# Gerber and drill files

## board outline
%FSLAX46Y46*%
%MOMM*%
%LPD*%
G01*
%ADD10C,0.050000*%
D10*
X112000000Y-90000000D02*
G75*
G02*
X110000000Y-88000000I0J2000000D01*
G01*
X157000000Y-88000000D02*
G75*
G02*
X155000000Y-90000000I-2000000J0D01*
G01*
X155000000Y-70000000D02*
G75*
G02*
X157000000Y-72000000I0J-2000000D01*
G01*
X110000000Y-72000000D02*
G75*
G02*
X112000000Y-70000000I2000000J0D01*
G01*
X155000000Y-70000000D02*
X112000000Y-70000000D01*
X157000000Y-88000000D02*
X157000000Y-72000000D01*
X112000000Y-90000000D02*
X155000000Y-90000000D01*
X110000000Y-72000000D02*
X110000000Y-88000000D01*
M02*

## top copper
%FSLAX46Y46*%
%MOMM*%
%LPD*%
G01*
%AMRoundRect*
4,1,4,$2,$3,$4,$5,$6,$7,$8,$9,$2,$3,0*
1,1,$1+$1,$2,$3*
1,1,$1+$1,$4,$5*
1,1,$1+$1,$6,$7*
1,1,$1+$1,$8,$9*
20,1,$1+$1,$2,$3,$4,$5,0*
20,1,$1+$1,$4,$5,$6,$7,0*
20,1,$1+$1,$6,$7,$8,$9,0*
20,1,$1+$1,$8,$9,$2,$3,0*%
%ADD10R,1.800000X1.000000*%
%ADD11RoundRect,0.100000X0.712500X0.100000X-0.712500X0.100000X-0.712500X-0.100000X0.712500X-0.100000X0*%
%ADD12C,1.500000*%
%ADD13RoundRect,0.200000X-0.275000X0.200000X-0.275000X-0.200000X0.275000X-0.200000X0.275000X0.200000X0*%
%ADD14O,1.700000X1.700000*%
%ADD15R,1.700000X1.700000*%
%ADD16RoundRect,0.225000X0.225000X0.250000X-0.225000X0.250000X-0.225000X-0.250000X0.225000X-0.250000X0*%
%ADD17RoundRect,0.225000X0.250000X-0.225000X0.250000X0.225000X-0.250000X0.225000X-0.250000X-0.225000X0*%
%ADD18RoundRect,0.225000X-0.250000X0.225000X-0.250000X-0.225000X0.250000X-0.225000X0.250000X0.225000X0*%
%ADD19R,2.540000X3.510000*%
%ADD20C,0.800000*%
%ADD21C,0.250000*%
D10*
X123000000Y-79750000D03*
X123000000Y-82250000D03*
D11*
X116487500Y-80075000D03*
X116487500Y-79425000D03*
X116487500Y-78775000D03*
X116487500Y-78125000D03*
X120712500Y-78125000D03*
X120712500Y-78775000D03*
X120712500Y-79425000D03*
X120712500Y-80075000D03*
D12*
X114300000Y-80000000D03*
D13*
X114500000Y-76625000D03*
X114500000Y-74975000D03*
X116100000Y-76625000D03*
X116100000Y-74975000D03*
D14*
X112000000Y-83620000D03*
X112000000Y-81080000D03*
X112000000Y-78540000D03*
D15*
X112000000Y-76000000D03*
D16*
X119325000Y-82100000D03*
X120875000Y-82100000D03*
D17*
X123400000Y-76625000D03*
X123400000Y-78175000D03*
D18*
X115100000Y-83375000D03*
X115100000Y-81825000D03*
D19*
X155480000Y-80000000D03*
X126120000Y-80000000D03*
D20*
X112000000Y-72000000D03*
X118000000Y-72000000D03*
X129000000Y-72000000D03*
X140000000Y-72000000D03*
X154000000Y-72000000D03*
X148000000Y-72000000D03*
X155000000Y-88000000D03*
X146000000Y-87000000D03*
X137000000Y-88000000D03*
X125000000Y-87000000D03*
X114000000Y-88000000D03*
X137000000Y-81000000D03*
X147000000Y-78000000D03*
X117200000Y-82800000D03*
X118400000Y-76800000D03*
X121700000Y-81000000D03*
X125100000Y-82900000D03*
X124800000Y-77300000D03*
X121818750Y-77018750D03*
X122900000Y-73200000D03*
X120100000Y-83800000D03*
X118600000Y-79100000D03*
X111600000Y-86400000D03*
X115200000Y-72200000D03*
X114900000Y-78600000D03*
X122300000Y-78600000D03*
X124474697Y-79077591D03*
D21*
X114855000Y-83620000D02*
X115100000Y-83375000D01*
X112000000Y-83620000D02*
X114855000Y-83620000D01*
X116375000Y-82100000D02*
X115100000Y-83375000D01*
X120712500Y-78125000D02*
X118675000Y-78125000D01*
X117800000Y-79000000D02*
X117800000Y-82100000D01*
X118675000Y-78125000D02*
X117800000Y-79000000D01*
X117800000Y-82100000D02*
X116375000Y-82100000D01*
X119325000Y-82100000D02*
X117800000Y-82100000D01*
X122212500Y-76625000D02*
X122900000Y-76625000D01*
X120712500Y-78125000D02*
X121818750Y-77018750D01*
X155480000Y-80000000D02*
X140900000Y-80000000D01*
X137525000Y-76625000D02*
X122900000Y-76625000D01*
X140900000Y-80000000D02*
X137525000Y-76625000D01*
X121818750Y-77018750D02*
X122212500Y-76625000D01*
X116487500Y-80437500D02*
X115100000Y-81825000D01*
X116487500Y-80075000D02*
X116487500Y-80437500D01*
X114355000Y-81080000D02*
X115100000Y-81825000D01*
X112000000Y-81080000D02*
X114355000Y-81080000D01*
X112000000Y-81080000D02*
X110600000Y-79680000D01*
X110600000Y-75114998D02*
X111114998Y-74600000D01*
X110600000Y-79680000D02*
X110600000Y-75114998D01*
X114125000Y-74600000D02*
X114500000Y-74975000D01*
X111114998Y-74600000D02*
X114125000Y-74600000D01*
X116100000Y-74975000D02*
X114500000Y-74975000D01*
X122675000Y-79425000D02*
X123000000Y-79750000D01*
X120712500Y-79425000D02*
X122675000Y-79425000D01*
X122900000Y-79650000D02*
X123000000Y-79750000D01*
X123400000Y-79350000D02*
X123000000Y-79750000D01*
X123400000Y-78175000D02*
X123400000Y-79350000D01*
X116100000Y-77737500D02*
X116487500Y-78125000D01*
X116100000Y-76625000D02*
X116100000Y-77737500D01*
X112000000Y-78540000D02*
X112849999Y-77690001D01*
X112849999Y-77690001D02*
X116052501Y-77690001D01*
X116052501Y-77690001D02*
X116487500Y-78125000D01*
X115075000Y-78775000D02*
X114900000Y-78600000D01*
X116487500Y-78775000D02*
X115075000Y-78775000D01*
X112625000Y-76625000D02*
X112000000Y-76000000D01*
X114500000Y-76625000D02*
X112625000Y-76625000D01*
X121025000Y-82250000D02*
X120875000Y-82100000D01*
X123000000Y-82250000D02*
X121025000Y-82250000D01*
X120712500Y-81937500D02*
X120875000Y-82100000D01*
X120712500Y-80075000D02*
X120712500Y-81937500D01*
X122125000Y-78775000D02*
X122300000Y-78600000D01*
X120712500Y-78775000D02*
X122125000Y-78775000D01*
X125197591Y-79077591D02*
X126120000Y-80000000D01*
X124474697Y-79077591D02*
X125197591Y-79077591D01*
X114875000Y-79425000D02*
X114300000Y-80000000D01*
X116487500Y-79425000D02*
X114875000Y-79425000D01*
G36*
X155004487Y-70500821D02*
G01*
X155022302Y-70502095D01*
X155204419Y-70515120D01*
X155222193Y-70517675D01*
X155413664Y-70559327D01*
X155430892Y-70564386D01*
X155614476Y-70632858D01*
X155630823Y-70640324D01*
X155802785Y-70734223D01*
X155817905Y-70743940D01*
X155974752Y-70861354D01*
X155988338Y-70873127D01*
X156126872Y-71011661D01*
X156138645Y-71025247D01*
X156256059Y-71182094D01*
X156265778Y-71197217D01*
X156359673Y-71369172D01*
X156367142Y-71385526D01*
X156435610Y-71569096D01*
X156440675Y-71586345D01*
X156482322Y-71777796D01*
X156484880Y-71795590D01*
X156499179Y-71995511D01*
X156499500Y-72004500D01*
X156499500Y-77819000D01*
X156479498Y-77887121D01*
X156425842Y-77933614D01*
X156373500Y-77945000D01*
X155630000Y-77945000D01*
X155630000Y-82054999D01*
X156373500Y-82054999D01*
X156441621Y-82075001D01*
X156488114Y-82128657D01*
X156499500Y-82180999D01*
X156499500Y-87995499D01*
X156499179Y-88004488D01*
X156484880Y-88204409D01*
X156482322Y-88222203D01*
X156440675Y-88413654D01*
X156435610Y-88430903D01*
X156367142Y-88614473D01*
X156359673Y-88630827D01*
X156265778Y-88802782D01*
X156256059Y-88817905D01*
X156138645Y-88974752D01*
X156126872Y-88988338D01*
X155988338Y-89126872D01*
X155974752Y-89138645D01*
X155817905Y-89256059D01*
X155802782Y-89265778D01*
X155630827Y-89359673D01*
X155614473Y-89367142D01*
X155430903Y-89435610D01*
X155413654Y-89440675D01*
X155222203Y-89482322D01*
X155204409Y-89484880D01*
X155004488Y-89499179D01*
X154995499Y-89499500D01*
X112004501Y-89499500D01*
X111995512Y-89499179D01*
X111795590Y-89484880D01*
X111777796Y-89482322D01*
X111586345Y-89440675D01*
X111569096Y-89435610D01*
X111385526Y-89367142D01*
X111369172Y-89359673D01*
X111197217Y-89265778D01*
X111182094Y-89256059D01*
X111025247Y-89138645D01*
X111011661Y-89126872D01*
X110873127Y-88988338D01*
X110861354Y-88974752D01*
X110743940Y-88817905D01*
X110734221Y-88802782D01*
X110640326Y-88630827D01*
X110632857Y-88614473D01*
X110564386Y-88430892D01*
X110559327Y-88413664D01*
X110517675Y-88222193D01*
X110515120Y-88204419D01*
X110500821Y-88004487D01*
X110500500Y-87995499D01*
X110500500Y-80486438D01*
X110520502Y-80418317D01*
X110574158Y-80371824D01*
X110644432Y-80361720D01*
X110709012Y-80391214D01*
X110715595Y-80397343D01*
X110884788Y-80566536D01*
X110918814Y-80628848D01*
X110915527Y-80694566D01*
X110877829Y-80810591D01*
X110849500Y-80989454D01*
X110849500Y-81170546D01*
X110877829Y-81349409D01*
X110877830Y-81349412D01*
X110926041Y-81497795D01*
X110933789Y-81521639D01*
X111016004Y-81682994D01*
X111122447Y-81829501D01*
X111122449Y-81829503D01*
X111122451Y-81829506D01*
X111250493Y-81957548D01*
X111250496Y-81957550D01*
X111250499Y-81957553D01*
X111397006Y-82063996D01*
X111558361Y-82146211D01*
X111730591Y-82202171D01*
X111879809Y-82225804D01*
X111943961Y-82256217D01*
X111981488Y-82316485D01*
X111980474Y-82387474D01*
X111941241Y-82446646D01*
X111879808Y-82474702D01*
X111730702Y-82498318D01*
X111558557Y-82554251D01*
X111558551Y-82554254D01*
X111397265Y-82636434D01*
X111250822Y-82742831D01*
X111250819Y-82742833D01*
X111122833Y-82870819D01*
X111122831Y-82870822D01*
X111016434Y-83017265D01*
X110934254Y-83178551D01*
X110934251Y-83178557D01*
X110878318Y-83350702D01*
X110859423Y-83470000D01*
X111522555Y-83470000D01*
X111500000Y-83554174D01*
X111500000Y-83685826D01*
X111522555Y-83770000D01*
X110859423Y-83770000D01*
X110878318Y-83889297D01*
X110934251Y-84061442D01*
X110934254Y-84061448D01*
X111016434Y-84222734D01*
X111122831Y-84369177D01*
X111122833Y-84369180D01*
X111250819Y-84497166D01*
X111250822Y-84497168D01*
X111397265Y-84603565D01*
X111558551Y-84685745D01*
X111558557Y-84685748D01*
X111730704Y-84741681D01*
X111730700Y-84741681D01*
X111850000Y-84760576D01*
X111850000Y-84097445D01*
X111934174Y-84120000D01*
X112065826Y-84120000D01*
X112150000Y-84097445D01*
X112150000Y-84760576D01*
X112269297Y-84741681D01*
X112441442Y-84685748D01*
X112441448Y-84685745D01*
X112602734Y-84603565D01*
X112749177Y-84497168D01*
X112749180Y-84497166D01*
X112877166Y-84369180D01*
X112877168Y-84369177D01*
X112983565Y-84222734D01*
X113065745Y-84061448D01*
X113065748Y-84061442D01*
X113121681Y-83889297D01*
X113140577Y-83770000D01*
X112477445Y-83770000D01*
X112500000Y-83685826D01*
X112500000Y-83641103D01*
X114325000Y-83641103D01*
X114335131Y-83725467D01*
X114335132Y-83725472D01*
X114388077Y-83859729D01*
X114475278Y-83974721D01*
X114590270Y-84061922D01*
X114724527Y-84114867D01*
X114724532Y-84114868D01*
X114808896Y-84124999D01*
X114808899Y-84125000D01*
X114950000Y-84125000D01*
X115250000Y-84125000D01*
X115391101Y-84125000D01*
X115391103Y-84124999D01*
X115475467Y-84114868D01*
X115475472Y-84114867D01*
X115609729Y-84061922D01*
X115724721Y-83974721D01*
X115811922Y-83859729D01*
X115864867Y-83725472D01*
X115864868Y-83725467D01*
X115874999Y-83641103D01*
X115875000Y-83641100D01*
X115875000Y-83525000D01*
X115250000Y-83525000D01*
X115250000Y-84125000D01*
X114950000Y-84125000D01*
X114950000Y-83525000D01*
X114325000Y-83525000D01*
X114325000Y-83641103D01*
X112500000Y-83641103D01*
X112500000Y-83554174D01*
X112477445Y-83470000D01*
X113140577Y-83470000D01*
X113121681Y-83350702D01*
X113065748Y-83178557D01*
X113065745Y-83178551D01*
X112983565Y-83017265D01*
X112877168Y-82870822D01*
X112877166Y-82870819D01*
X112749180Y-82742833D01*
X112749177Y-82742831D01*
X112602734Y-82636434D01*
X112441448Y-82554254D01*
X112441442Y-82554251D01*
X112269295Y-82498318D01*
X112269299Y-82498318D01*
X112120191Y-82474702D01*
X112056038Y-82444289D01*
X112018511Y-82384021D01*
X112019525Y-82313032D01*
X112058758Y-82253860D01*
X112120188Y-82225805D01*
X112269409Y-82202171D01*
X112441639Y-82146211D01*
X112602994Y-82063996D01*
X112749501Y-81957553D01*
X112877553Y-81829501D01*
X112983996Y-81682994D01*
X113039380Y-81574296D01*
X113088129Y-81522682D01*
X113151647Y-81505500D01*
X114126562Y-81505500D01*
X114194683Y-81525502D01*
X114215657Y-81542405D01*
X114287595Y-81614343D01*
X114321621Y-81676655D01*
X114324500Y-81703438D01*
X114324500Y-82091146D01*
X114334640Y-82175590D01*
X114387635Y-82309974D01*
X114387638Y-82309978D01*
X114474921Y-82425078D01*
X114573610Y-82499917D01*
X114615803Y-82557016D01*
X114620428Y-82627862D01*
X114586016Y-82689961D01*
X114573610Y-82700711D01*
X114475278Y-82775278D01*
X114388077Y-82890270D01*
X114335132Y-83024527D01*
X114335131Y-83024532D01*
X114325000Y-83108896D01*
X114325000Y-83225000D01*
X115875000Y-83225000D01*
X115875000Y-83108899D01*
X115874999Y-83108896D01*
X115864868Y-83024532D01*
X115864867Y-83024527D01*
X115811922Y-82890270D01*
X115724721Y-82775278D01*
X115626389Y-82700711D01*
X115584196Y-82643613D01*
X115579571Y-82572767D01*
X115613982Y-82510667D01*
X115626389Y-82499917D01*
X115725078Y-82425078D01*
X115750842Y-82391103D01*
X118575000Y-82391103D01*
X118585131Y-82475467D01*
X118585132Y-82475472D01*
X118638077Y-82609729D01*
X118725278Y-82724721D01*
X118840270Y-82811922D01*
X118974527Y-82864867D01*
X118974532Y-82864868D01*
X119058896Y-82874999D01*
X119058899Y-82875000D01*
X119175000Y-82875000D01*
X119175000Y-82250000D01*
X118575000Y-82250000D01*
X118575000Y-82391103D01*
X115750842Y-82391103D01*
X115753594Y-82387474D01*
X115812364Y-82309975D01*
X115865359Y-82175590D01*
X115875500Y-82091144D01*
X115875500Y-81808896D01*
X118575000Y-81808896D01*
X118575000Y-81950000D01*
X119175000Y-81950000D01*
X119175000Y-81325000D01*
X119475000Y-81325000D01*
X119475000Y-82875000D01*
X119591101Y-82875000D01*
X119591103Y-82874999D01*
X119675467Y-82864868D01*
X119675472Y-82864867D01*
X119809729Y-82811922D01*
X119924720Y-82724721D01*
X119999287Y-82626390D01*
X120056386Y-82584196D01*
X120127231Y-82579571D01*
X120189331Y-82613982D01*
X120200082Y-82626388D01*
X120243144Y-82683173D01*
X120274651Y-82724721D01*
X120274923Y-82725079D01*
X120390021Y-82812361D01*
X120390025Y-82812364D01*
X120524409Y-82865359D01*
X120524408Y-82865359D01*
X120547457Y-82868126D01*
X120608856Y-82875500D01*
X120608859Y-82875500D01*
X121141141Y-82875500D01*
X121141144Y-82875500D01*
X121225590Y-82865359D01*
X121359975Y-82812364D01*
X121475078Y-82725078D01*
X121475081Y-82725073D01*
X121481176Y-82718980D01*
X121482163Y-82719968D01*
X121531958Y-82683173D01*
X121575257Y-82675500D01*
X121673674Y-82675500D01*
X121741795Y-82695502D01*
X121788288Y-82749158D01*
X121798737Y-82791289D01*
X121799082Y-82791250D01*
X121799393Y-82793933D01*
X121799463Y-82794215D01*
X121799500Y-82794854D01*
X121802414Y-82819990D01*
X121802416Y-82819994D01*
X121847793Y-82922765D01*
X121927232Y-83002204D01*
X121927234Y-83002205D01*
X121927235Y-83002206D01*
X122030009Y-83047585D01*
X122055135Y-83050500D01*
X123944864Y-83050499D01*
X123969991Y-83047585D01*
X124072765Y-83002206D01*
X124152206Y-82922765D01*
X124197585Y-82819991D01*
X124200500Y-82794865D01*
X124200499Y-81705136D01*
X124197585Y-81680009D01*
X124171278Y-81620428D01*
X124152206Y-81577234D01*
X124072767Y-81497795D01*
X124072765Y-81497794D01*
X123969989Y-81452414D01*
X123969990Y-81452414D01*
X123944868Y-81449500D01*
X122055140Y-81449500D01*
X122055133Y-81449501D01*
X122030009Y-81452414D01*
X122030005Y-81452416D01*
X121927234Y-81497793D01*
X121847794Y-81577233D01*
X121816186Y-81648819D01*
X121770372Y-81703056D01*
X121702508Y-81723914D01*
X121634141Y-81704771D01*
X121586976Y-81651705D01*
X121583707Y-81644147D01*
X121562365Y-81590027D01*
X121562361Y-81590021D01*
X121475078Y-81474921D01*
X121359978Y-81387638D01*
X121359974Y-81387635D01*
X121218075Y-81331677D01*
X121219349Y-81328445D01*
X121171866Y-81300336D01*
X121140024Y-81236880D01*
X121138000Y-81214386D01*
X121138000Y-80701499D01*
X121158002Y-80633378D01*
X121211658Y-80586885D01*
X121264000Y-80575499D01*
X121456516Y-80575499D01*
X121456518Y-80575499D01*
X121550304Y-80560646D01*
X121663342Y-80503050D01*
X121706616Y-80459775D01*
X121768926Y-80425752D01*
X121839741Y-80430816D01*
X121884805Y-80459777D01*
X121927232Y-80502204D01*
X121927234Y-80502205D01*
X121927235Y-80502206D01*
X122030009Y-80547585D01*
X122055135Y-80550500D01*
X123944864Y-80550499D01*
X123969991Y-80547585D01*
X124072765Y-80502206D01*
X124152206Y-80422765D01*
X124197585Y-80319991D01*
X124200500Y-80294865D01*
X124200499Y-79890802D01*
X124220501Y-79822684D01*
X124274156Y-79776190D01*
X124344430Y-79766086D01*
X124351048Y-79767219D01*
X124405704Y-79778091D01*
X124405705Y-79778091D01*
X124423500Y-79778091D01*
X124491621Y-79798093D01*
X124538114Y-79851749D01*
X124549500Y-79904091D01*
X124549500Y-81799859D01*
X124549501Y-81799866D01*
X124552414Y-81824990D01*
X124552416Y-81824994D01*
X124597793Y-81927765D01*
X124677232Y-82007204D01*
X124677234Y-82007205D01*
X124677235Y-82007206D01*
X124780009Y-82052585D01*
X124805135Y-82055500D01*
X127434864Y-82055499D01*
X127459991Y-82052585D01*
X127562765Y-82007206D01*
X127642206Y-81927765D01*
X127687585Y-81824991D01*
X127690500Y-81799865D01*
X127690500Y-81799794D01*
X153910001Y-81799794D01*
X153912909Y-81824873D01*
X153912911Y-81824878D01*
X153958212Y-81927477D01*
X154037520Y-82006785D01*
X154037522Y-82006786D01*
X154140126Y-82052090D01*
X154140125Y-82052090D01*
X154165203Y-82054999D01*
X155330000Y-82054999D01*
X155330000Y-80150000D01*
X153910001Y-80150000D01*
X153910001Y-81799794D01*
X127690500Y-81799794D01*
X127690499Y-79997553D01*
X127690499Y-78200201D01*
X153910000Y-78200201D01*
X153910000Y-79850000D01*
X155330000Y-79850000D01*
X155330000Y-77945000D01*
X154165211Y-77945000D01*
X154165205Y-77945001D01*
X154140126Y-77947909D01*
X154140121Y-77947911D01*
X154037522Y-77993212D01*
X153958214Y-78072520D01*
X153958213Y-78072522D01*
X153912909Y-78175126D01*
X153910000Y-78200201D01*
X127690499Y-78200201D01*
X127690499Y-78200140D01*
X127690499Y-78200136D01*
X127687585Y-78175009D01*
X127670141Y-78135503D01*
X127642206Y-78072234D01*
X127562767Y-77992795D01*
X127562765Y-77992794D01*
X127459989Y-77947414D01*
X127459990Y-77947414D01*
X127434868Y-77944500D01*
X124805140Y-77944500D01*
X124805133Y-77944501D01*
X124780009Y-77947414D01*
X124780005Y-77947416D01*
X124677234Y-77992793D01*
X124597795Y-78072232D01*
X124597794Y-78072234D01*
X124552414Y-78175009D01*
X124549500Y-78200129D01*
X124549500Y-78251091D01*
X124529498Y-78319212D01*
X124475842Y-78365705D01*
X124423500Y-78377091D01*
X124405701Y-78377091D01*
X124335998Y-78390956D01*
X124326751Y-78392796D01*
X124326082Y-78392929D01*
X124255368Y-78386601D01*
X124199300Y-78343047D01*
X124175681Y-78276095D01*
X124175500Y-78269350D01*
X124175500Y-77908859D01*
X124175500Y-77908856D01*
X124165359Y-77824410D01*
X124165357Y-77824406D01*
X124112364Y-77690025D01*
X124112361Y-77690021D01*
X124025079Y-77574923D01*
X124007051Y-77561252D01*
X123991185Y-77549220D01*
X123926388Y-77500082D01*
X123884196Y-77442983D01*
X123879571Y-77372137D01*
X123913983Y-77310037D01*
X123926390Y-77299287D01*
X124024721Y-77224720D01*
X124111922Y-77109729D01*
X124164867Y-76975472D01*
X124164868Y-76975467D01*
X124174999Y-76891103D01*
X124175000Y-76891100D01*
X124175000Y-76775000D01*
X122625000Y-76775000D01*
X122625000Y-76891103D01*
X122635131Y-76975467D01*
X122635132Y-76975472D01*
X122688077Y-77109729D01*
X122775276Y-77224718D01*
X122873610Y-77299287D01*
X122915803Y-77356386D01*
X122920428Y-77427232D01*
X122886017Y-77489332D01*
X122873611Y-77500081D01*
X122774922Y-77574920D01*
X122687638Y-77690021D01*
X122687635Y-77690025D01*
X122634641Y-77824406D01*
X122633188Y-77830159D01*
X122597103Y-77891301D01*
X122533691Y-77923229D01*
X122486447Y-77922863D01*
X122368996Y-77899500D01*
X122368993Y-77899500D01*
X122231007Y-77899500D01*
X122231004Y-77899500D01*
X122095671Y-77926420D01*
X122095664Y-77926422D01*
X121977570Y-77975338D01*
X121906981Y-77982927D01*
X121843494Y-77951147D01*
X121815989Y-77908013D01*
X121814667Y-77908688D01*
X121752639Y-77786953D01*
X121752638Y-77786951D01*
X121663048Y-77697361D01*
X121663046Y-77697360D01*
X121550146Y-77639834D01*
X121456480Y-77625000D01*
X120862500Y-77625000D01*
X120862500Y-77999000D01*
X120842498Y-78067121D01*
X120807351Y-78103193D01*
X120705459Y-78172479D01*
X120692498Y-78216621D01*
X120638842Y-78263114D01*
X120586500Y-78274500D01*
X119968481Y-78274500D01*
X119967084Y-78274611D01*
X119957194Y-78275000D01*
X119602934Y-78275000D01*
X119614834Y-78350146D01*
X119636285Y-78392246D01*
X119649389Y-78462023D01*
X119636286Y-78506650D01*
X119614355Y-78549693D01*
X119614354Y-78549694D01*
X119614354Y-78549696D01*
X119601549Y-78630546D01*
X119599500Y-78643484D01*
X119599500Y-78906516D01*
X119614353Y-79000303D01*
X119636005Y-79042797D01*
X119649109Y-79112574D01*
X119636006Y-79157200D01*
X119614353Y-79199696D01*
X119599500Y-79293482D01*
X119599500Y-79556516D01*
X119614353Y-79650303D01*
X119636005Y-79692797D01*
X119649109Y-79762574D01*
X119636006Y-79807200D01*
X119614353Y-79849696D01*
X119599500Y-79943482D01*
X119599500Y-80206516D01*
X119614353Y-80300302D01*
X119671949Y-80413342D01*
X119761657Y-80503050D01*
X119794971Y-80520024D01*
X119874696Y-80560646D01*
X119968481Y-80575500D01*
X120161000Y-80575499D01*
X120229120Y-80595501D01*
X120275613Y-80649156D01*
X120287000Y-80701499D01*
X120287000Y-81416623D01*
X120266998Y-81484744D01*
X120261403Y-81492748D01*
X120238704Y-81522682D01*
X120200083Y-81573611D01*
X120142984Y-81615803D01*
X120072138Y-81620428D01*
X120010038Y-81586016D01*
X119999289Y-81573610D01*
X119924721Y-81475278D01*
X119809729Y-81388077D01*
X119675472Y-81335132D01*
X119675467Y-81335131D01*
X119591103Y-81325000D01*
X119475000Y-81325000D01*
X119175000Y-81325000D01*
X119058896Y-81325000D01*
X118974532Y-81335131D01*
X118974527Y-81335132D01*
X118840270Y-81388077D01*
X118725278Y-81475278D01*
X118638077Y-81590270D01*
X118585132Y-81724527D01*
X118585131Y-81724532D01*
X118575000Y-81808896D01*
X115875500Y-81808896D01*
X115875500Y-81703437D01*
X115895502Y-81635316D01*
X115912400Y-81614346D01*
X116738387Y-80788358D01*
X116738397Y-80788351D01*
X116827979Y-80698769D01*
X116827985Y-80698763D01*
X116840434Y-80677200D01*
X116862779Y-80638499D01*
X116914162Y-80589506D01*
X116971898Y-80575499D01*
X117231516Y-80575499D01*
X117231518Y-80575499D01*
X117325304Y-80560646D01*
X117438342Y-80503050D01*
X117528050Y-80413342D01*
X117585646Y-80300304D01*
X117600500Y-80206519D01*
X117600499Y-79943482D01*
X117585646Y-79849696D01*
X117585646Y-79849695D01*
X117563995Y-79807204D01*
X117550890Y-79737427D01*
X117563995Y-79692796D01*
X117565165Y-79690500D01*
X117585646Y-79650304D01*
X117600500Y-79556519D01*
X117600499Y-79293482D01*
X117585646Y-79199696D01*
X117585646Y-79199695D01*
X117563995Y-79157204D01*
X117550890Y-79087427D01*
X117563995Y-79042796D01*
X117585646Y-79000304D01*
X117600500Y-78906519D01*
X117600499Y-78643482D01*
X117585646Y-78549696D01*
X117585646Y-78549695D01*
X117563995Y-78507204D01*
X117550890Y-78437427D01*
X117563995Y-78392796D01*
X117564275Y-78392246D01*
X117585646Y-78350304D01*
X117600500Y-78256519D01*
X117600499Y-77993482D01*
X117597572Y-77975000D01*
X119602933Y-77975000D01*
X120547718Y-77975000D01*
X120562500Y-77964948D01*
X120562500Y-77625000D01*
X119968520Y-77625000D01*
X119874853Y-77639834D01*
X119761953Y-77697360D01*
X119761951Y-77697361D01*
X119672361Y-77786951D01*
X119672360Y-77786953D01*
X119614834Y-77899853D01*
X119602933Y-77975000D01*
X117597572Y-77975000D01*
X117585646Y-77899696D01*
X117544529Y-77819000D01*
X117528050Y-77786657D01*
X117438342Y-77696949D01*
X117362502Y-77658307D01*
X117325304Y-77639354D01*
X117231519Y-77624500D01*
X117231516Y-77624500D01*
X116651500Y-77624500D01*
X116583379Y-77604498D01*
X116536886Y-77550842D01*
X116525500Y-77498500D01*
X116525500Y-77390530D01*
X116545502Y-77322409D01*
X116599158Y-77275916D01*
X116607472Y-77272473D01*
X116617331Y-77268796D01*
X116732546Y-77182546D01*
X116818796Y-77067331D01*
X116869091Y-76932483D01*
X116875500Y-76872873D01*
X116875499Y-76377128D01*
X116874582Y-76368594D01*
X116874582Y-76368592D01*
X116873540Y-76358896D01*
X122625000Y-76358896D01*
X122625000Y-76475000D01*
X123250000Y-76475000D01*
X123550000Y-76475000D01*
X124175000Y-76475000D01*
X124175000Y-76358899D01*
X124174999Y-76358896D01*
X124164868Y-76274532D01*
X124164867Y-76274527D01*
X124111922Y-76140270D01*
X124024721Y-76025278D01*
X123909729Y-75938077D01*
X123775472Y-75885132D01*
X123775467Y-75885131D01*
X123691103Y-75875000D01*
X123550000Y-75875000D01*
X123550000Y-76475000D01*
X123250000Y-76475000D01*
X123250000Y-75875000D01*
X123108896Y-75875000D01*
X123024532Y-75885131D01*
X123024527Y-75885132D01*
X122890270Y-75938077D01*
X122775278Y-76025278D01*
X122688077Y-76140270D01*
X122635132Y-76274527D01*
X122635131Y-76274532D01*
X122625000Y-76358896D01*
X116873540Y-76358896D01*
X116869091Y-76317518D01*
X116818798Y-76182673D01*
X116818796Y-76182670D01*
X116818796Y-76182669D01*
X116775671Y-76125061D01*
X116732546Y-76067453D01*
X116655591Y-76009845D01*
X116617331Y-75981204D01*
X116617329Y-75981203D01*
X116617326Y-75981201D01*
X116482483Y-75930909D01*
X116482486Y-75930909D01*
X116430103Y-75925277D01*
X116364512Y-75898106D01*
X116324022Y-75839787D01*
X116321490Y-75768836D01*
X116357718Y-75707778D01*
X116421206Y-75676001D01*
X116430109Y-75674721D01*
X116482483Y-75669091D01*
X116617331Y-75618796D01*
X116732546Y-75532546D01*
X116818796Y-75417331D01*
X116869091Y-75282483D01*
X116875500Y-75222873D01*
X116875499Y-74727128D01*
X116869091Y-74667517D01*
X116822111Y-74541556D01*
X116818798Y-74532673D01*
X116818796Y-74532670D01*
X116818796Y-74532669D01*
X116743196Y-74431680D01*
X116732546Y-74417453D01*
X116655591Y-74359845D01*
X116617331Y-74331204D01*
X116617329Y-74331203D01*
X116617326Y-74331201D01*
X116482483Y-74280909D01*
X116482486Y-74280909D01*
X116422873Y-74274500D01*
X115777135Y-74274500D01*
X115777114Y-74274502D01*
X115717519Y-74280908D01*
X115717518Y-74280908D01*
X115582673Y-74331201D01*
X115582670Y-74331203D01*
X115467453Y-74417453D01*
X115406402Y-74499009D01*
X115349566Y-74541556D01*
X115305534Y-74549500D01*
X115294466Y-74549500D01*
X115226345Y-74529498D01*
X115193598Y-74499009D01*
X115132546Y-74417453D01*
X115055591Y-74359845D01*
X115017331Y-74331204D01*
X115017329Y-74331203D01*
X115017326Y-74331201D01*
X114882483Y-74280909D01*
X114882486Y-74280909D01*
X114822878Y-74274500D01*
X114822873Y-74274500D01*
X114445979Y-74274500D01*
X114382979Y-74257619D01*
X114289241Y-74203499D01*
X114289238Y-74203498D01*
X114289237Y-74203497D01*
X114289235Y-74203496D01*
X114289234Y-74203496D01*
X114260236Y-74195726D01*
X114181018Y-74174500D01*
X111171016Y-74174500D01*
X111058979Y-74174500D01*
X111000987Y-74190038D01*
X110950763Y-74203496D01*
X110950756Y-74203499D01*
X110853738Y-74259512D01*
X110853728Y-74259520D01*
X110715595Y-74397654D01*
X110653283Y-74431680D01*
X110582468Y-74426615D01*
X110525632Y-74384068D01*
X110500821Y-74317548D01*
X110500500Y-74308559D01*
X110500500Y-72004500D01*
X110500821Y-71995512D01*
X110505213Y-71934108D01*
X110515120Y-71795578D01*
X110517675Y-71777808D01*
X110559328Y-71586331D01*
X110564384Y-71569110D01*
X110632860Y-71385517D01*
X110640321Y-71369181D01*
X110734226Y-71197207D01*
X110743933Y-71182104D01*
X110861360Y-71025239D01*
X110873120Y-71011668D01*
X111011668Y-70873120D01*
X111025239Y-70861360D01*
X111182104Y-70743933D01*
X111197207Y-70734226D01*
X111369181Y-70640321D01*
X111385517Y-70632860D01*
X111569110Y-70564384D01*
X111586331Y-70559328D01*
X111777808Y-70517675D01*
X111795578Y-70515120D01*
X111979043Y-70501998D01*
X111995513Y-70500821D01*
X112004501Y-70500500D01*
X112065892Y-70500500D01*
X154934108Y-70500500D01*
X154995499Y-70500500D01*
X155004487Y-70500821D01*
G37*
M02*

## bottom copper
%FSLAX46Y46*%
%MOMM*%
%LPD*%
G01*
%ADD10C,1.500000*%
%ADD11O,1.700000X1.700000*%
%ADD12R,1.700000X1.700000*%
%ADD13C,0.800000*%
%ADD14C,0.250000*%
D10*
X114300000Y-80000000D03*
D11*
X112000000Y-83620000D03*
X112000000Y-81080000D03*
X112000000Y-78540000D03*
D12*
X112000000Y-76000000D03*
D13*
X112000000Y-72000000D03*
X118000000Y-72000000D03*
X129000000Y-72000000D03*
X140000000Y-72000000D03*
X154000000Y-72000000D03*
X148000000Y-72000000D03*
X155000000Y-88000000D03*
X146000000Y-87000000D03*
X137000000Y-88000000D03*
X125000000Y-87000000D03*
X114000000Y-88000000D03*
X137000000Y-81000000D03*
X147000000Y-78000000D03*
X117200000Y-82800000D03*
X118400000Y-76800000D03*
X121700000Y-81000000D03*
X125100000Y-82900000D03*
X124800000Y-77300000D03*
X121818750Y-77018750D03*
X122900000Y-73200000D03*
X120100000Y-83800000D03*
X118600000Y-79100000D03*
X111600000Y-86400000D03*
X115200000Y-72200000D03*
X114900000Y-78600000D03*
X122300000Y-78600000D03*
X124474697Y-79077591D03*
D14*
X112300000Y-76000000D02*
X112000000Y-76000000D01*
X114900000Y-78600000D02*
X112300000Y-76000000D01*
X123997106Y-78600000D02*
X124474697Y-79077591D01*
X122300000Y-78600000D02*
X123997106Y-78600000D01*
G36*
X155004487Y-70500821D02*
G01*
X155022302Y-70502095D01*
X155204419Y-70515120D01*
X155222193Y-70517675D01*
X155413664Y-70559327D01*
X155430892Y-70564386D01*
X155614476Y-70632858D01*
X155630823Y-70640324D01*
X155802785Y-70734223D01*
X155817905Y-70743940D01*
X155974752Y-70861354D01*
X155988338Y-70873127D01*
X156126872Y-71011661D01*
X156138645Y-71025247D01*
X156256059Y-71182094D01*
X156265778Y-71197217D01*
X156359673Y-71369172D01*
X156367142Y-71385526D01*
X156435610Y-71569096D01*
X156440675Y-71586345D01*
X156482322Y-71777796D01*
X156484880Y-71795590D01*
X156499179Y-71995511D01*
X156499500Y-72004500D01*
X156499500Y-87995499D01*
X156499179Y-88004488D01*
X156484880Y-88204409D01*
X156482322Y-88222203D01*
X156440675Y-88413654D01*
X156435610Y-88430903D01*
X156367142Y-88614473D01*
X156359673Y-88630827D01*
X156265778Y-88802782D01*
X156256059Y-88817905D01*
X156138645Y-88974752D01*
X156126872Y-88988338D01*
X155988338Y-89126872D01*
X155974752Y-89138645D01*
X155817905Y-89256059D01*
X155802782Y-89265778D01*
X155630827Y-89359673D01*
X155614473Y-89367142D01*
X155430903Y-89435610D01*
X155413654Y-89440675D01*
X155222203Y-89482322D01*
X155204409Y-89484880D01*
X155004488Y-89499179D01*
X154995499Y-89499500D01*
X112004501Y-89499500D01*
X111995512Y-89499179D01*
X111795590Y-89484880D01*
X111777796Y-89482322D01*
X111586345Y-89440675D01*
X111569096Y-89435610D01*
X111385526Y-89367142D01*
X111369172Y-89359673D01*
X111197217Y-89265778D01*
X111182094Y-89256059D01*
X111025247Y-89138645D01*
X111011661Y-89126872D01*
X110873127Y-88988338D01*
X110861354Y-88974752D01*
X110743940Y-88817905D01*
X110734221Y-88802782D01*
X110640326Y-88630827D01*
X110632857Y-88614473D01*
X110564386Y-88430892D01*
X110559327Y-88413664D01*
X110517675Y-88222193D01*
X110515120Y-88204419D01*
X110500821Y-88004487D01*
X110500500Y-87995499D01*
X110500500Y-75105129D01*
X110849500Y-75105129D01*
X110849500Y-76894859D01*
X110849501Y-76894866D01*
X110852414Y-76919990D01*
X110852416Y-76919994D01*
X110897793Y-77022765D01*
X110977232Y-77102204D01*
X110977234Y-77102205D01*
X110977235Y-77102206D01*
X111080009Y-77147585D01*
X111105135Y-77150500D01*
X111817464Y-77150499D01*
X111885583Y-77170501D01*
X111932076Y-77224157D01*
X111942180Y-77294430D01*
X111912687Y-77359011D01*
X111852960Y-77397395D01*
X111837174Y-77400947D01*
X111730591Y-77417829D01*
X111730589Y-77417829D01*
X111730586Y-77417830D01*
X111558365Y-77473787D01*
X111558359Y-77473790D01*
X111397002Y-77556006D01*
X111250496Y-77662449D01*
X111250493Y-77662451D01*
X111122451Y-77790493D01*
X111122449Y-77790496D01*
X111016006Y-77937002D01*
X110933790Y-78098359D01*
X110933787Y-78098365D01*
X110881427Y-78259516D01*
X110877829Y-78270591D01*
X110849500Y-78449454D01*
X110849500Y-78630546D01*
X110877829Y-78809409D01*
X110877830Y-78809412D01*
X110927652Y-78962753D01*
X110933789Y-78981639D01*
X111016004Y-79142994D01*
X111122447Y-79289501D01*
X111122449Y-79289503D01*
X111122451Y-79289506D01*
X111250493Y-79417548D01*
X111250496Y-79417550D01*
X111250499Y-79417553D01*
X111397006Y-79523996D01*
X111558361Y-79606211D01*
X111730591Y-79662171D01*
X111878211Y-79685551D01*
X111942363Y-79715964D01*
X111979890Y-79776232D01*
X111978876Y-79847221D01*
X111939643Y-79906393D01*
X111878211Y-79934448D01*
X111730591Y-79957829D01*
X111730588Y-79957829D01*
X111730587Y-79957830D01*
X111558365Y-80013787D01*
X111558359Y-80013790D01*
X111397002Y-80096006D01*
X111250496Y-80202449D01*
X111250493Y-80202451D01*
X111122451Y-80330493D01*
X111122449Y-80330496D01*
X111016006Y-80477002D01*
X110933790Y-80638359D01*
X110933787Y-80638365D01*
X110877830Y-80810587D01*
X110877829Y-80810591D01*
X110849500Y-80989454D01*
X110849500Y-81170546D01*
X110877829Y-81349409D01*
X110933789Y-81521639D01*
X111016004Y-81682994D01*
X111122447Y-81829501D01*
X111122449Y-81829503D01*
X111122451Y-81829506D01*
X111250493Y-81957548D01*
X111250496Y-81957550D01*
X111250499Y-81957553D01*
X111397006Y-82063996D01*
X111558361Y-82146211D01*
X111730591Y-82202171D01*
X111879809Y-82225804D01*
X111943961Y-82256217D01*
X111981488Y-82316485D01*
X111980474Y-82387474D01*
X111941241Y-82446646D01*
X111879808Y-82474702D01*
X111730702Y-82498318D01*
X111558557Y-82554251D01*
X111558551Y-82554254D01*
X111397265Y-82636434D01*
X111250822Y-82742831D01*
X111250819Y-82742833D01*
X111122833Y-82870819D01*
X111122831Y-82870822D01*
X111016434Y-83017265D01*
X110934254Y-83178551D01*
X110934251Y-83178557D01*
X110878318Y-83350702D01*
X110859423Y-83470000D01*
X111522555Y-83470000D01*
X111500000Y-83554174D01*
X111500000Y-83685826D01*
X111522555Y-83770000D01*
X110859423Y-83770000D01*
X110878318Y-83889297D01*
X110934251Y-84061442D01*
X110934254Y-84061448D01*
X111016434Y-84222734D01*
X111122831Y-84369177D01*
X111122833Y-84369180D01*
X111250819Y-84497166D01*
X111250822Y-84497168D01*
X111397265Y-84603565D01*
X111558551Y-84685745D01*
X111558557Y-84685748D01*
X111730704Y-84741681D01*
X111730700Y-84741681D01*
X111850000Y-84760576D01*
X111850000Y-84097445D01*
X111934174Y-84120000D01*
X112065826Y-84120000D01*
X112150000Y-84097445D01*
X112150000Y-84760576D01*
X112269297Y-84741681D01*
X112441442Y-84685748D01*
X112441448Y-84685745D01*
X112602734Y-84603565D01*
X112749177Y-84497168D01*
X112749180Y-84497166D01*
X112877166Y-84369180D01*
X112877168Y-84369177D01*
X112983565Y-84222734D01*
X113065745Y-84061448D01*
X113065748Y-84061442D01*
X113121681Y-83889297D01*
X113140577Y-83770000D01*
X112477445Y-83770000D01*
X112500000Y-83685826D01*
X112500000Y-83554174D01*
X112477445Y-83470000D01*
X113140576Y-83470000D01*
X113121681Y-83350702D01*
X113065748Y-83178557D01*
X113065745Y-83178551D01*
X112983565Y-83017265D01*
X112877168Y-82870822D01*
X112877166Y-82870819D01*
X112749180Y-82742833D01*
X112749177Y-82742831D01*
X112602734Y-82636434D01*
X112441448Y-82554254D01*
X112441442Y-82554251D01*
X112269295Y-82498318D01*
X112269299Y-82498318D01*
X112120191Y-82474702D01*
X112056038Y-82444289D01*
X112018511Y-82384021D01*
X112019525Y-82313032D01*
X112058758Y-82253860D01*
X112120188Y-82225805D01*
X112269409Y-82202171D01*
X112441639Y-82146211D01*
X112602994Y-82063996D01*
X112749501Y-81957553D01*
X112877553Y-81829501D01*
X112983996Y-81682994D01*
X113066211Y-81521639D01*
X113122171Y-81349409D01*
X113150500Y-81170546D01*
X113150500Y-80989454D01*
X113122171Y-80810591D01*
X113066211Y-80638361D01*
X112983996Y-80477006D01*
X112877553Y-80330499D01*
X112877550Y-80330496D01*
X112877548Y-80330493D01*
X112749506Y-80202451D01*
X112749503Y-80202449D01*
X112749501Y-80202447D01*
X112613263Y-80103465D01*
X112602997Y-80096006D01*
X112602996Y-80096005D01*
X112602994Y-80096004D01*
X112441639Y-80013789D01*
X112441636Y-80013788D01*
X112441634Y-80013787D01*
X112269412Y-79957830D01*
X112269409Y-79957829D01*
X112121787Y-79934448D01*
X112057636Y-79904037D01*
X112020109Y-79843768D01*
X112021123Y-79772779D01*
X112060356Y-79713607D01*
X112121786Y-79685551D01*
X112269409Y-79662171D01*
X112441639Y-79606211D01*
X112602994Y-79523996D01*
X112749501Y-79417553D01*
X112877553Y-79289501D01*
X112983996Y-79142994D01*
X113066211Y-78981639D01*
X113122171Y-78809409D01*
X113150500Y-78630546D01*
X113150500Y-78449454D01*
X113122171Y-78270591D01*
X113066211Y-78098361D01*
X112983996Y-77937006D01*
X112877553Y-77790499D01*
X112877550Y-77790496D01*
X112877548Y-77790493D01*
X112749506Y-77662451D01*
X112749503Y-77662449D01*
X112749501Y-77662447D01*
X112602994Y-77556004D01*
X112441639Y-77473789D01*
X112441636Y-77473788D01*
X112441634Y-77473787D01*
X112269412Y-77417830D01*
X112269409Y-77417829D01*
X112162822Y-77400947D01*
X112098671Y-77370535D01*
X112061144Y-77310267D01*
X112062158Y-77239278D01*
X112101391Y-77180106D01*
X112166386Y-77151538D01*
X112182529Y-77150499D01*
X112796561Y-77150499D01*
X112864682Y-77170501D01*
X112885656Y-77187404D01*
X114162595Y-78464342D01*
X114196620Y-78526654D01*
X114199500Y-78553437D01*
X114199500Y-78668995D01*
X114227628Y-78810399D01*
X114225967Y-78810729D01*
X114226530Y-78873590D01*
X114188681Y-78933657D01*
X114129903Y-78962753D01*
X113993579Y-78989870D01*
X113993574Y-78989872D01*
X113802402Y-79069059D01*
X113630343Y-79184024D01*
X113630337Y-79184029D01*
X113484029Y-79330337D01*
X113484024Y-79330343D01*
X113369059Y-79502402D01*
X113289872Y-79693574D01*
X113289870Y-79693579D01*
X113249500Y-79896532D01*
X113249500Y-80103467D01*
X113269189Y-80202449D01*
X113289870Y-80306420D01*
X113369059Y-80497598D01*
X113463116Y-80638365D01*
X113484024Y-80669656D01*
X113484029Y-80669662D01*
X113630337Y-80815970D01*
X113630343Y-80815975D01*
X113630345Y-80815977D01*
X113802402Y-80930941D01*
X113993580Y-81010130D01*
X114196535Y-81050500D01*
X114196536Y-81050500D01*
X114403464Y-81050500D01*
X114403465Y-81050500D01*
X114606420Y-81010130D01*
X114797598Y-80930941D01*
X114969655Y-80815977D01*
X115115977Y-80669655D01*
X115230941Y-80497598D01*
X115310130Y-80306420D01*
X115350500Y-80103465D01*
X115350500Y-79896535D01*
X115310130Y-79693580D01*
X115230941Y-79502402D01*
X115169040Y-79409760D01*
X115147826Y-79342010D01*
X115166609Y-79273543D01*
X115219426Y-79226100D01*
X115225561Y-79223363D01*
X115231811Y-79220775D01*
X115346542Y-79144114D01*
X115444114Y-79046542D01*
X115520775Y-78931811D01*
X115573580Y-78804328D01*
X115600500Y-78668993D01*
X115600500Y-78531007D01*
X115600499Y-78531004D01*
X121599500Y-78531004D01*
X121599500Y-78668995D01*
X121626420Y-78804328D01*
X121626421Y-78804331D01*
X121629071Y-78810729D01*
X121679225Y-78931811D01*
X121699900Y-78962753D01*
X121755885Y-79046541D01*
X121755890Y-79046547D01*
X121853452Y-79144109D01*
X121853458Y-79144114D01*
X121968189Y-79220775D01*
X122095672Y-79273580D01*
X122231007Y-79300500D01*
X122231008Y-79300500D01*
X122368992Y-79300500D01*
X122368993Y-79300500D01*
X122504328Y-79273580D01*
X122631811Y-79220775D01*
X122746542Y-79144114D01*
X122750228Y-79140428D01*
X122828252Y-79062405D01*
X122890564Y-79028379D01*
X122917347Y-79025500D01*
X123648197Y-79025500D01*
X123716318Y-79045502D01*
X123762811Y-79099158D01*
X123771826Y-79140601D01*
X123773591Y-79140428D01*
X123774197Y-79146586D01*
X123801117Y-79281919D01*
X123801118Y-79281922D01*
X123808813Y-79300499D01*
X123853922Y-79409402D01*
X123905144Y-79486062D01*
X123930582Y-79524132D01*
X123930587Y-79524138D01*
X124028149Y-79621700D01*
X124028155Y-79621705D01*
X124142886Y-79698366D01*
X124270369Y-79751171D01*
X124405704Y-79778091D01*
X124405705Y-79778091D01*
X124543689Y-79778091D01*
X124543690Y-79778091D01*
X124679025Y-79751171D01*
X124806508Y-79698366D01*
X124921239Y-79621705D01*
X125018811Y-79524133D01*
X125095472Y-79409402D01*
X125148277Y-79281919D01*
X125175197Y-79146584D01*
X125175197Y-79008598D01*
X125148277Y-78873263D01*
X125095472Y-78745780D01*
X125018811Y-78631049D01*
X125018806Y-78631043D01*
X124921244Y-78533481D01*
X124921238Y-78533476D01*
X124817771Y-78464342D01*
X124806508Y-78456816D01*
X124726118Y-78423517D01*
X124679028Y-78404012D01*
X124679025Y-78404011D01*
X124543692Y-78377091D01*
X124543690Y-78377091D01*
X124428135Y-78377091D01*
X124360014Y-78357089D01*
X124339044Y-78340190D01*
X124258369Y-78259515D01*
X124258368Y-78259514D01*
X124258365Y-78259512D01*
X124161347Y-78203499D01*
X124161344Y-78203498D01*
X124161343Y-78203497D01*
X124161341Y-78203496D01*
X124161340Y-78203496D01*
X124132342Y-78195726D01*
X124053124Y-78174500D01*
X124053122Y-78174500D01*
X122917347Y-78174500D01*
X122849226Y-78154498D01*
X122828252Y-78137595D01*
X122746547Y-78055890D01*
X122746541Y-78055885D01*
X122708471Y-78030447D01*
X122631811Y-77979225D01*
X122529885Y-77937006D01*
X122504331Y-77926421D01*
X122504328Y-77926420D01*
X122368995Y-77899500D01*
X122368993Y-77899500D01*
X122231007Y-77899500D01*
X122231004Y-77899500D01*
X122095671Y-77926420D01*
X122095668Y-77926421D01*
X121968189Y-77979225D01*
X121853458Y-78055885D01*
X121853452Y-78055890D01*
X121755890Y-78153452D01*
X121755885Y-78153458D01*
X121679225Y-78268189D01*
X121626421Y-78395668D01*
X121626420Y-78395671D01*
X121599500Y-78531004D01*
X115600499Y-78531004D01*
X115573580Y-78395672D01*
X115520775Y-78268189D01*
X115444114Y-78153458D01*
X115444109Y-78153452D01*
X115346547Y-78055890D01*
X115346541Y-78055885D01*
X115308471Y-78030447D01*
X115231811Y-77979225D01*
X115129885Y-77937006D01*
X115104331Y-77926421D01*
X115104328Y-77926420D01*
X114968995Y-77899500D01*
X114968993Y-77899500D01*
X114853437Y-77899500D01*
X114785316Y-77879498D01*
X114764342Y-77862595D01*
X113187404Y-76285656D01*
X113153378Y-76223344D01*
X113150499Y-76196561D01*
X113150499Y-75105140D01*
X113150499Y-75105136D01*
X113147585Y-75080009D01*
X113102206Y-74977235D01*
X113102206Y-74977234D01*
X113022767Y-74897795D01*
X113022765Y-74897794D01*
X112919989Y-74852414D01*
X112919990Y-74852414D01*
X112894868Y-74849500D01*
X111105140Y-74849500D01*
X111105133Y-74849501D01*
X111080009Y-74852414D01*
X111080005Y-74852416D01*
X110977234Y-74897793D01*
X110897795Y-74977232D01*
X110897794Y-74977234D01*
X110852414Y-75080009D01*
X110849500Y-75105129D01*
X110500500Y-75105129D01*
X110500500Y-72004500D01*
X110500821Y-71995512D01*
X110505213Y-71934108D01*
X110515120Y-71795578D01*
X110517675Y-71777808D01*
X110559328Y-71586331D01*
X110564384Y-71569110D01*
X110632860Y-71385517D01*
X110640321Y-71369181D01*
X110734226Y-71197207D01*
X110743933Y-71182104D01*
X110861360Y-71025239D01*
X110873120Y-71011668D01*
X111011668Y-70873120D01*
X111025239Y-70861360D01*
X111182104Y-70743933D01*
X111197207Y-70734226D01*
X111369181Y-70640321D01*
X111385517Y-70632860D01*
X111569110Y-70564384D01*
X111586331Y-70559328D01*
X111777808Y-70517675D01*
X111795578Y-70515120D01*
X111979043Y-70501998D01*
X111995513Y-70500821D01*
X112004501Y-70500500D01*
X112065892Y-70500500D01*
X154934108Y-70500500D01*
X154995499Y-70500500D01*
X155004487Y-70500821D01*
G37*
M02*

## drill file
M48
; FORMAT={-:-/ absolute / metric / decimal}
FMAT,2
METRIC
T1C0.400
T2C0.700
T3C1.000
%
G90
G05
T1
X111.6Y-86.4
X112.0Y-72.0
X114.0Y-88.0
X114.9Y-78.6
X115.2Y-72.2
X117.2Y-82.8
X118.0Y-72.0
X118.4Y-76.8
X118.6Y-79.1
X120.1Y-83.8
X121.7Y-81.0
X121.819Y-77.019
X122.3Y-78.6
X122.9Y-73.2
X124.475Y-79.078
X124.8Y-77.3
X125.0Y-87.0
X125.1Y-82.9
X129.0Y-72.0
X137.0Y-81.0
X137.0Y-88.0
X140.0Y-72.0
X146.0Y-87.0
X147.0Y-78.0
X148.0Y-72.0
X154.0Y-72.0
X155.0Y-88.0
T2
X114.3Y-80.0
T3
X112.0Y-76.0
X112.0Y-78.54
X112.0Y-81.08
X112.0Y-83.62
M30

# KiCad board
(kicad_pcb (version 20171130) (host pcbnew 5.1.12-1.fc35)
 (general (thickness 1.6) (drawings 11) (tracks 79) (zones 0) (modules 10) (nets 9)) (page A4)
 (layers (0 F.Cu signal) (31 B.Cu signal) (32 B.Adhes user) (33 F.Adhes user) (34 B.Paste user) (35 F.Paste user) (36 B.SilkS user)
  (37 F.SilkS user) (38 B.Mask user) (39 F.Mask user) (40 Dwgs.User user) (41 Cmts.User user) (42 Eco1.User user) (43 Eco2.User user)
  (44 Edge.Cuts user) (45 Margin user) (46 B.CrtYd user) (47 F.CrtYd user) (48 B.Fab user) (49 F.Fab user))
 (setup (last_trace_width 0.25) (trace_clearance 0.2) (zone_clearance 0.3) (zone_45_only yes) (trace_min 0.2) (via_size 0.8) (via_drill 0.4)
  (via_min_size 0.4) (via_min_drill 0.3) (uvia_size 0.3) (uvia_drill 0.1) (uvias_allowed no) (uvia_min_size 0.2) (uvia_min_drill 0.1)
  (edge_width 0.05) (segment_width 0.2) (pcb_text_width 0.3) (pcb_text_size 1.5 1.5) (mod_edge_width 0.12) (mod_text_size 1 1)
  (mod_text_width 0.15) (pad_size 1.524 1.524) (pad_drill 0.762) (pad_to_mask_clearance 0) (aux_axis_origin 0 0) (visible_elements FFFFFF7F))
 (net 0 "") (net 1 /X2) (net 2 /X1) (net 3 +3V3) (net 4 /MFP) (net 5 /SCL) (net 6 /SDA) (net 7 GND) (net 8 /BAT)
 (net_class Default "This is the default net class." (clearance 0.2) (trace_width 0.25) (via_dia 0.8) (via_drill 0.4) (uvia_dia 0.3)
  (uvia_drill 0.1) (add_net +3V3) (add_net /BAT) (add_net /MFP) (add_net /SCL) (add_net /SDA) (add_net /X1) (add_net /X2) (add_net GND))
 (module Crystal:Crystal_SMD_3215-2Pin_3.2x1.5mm (layer F.Cu) (at 123 81 270)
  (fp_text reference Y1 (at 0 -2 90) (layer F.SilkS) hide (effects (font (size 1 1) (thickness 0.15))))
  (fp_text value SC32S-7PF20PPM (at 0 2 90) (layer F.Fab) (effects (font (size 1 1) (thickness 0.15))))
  (pad 2 smd rect (at -1.25 0 270) (size 1 1.8) (layers F.Cu F.Paste F.Mask) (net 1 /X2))
  (pad 1 smd rect (at 1.25 0 270) (size 1 1.8) (layers F.Cu F.Paste F.Mask) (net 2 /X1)))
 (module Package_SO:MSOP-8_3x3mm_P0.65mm (layer F.Cu) (at 118.6 79.1 180)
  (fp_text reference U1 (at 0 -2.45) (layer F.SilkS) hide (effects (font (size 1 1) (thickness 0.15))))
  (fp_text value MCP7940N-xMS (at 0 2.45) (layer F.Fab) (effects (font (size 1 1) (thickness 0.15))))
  (pad 8 smd roundrect (at 2.1125 -0.975 180) (size 1.625 0.4) (layers F.Cu F.Paste F.Mask) (roundrect_rratio 0.25) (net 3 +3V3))
  (pad 7 smd roundrect (at 2.1125 -0.325 180) (size 1.625 0.4) (layers F.Cu F.Paste F.Mask) (roundrect_rratio 0.25) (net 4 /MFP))
  (pad 6 smd roundrect (at 2.1125 0.325 180) (size 1.625 0.4) (layers F.Cu F.Paste F.Mask) (roundrect_rratio 0.25) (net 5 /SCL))
  (pad 5 smd roundrect (at 2.1125 0.975 180) (size 1.625 0.4) (layers F.Cu F.Paste F.Mask) (roundrect_rratio 0.25) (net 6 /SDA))
  (pad 4 smd roundrect (at -2.1125 0.975 180) (size 1.625 0.4) (layers F.Cu F.Paste F.Mask) (roundrect_rratio 0.25) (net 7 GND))
  (pad 3 smd roundrect (at -2.1125 0.325 180) (size 1.625 0.4) (layers F.Cu F.Paste F.Mask) (roundrect_rratio 0.25) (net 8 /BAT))
  (pad 2 smd roundrect (at -2.1125 -0.325 180) (size 1.625 0.4) (layers F.Cu F.Paste F.Mask) (roundrect_rratio 0.25) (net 1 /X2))
  (pad 1 smd roundrect (at -2.1125 -0.975 180) (size 1.625 0.4) (layers F.Cu F.Paste F.Mask) (roundrect_rratio 0.25) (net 2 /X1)))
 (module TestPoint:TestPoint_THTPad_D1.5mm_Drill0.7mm (layer F.Cu) (at 114.3 80)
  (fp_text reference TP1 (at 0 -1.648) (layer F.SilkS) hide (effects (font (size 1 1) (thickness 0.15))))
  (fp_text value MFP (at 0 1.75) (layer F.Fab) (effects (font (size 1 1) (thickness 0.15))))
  (pad 1 thru_hole circle (at 0 0) (size 1.5 1.5) (drill 0.7) (layers *.Cu *.Mask) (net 4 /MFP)))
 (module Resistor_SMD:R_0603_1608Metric (layer F.Cu) (at 114.5 75.8 270)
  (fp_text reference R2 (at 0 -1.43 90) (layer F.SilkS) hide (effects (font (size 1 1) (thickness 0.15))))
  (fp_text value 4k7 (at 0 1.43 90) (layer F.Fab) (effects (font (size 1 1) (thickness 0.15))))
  (pad 2 smd roundrect (at 0.825 0 270) (size 0.8 0.95) (layers F.Cu F.Paste F.Mask) (roundrect_rratio 0.25) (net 5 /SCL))
  (pad 1 smd roundrect (at -0.825 0 270) (size 0.8 0.95) (layers F.Cu F.Paste F.Mask) (roundrect_rratio 0.25) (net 3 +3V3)))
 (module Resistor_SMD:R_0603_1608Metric (layer F.Cu) (at 116.1 75.8 270)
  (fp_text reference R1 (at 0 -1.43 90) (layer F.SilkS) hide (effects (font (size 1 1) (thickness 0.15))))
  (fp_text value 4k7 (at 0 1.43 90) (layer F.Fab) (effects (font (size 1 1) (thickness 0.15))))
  (pad 2 smd roundrect (at 0.825 0 270) (size 0.8 0.95) (layers F.Cu F.Paste F.Mask) (roundrect_rratio 0.25) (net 6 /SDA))
  (pad 1 smd roundrect (at -0.825 0 270) (size 0.8 0.95) (layers F.Cu F.Paste F.Mask) (roundrect_rratio 0.25) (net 3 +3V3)))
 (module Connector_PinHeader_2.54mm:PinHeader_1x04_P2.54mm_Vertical (layer B.Cu) (at 112 76 180)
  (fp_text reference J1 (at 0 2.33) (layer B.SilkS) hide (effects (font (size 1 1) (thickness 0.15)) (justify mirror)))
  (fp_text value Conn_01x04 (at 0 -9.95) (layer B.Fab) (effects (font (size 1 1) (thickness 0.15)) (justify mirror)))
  (pad 4 thru_hole oval (at 0 -7.62 180) (size 1.7 1.7) (drill 1) (layers *.Cu *.Mask) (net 7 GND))
  (pad 3 thru_hole oval (at 0 -5.08 180) (size 1.7 1.7) (drill 1) (layers *.Cu *.Mask) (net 3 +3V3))
  (pad 2 thru_hole oval (at 0 -2.54 180) (size 1.7 1.7) (drill 1) (layers *.Cu *.Mask) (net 6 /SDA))
  (pad 1 thru_hole rect (at 0 0 180) (size 1.7 1.7) (drill 1) (layers *.Cu *.Mask) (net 5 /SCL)))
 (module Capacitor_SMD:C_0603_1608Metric (layer F.Cu) (at 120.1 82.1 180)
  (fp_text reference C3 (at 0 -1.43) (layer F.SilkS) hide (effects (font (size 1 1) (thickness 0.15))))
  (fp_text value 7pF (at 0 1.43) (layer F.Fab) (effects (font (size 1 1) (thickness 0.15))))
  (pad 2 smd roundrect (at 0.775 0 180) (size 0.9 0.95) (layers F.Cu F.Paste F.Mask) (roundrect_rratio 0.25) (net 7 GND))
  (pad 1 smd roundrect (at -0.775 0 180) (size 0.9 0.95) (layers F.Cu F.Paste F.Mask) (roundrect_rratio 0.25) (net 2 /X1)))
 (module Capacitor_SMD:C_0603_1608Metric (layer F.Cu) (at 123.4 77.4 90)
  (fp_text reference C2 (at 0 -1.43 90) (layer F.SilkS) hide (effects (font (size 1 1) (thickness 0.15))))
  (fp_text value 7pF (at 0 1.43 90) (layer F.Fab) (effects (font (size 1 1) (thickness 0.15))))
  (pad 2 smd roundrect (at 0.775 0 90) (size 0.9 0.95) (layers F.Cu F.Paste F.Mask) (roundrect_rratio 0.25) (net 7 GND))
  (pad 1 smd roundrect (at -0.775 0 90) (size 0.9 0.95) (layers F.Cu F.Paste F.Mask) (roundrect_rratio 0.25) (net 1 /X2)))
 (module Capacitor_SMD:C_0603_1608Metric (layer F.Cu) (at 115.1 82.6 270)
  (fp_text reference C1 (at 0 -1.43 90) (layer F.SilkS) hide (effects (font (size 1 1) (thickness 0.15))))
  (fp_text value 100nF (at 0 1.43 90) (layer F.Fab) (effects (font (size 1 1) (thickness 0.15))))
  (pad 2 smd roundrect (at 0.775 0 270) (size 0.9 0.95) (layers F.Cu F.Paste F.Mask) (roundrect_rratio 0.25) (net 7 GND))
  (pad 1 smd roundrect (at -0.775 0 270) (size 0.9 0.95) (layers F.Cu F.Paste F.Mask) (roundrect_rratio 0.25) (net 3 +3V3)))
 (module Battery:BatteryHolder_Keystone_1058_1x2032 (layer F.Cu) (at 140.8 80)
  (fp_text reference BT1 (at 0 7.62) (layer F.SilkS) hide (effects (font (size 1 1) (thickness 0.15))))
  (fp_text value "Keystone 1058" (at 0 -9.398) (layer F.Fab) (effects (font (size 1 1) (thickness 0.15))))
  (pad 2 smd rect (at 14.68 0) (size 2.54 3.51) (layers F.Cu F.Paste F.Mask) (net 7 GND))
  (pad 1 smd rect (at -14.68 0) (size 2.54 3.51) (layers F.Cu F.Paste F.Mask) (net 8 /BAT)))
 (gr_arc (start 112 88) (end 110 88) (angle -90) (layer Edge.Cuts) (width 0.05))
 (gr_arc (start 155 88) (end 155 90) (angle -90) (layer Edge.Cuts) (width 0.05))
 (gr_arc (start 155 72) (end 157 72) (angle -90) (layer Edge.Cuts) (width 0.05))
 (gr_arc (start 112 72) (end 112 70) (angle -90) (layer Edge.Cuts) (width 0.05))
 (gr_line (start 155 70) (end 112 70) (layer Edge.Cuts) (width 0.05))
 (gr_line (start 157 88) (end 157 72) (layer Edge.Cuts) (width 0.05))
 (gr_line (start 112 90) (end 155 90) (layer Edge.Cuts) (width 0.05))
 (gr_line (start 110 72) (end 110 88) (layer Edge.Cuts) (width 0.05))
 (segment (start 114.855 83.62) (end 115.1 83.375) (width 0.25) (layer F.Cu) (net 7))
 (segment (start 112 83.62) (end 114.855 83.62) (width 0.25) (layer F.Cu) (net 7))
 (segment (start 116.375 82.1) (end 115.1 83.375) (width 0.25) (layer F.Cu) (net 7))
 (segment (start 120.7125 78.125) (end 118.675 78.125) (width 0.25) (layer F.Cu) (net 7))
 (segment (start 117.8 79) (end 117.8 82.1) (width 0.25) (layer F.Cu) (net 7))
 (segment (start 118.675 78.125) (end 117.8 79) (width 0.25) (layer F.Cu) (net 7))
 (segment (start 117.8 82.1) (end 116.375 82.1) (width 0.25) (layer F.Cu) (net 7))
 (segment (start 119.325 82.1) (end 117.8 82.1) (width 0.25) (layer F.Cu) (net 7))
 (segment (start 122.2125 76.625) (end 122.9 76.625) (width 0.25) (layer F.Cu) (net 7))
 (segment (start 120.7125 78.125) (end 121.81875 77.01875) (width 0.25) (layer F.Cu) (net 7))
 (segment (start 155.48 80) (end 140.9 80) (width 0.25) (layer F.Cu) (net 7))
 (segment (start 137.525 76.625) (end 122.9 76.625) (width 0.25) (layer F.Cu) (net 7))
 (segment (start 140.9 80) (end 137.525 76.625) (width 0.25) (layer F.Cu) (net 7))
 (via (at 112 72) (size 0.8) (drill 0.4) (layers F.Cu B.Cu) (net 7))
 (via (at 118 72) (size 0.8) (drill 0.4) (layers F.Cu B.Cu) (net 7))
 (via (at 129 72) (size 0.8) (drill 0.4) (layers F.Cu B.Cu) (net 7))
 (via (at 140 72) (size 0.8) (drill 0.4) (layers F.Cu B.Cu) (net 7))
 (via (at 154 72) (size 0.8) (drill 0.4) (layers F.Cu B.Cu) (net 7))
 (via (at 148 72) (size 0.8) (drill 0.4) (layers F.Cu B.Cu) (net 7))
 (via (at 155 88) (size 0.8) (drill 0.4) (layers F.Cu B.Cu) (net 7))
 (via (at 146 87) (size 0.8) (drill 0.4) (layers F.Cu B.Cu) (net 7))
 (via (at 137 88) (size 0.8) (drill 0.4) (layers F.Cu B.Cu) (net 7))
 (via (at 125 87) (size 0.8) (drill 0.4) (layers F.Cu B.Cu) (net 7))
 (via (at 114 88) (size 0.8) (drill 0.4) (layers F.Cu B.Cu) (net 7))
 (via (at 137 81) (size 0.8) (drill 0.4) (layers F.Cu B.Cu) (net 7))
 (via (at 147 78) (size 0.8) (drill 0.4) (layers F.Cu B.Cu) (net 7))
 (via (at 117.2 82.8) (size 0.8) (drill 0.4) (layers F.Cu B.Cu) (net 7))
 (via (at 118.4 76.8) (size 0.8) (drill 0.4) (layers F.Cu B.Cu) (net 7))
 (via (at 121.7 81) (size 0.8) (drill 0.4) (layers F.Cu B.Cu) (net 7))
 (via (at 125.1 82.9) (size 0.8) (drill 0.4) (layers F.Cu B.Cu) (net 7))
 (via (at 124.8 77.3) (size 0.8) (drill 0.4) (layers F.Cu B.Cu) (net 7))
 (segment (start 121.81875 77.01875) (end 122.2125 76.625) (width 0.25) (layer F.Cu) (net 7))
 (via (at 121.81875 77.01875) (size 0.8) (drill 0.4) (layers F.Cu B.Cu) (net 7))
 (via (at 122.9 73.2) (size 0.8) (drill 0.4) (layers F.Cu B.Cu) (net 7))
 (via (at 120.1 83.8) (size 0.8) (drill 0.4) (layers F.Cu B.Cu) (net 7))
 (via (at 118.6 79.1) (size 0.8) (drill 0.4) (layers F.Cu B.Cu) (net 7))
 (via (at 111.6 86.4) (size 0.8) (drill 0.4) (layers F.Cu B.Cu) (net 7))
 (via (at 115.2 72.2) (size 0.8) (drill 0.4) (layers F.Cu B.Cu) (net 7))
 (segment (start 116.4875 80.4375) (end 115.1 81.825) (width 0.25) (layer F.Cu) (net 3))
 (segment (start 116.4875 80.075) (end 116.4875 80.4375) (width 0.25) (layer F.Cu) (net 3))
 (segment (start 114.355 81.08) (end 115.1 81.825) (width 0.25) (layer F.Cu) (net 3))
 (segment (start 112 81.08) (end 114.355 81.08) (width 0.25) (layer F.Cu) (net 3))
 (segment (start 112 81.08) (end 110.6 79.68) (width 0.25) (layer F.Cu) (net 3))
 (segment (start 110.6 75.114998) (end 111.114998 74.6) (width 0.25) (layer F.Cu) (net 3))
 (segment (start 110.6 79.68) (end 110.6 75.114998) (width 0.25) (layer F.Cu) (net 3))
 (segment (start 114.125 74.6) (end 114.5 74.975) (width 0.25) (layer F.Cu) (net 3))
 (segment (start 111.114998 74.6) (end 114.125 74.6) (width 0.25) (layer F.Cu) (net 3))
 (segment (start 116.1 74.975) (end 114.5 74.975) (width 0.25) (layer F.Cu) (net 3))
 (segment (start 122.675 79.425) (end 123 79.75) (width 0.25) (layer F.Cu) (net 1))
 (segment (start 120.7125 79.425) (end 122.675 79.425) (width 0.25) (layer F.Cu) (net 1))
 (segment (start 122.9 79.65) (end 123 79.75) (width 0.25) (layer F.Cu) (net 1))
 (segment (start 123.4 79.35) (end 123 79.75) (width 0.25) (layer F.Cu) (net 1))
 (segment (start 123.4 78.175) (end 123.4 79.35) (width 0.25) (layer F.Cu) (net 1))
 (segment (start 116.1 77.7375) (end 116.4875 78.125) (width 0.25) (layer F.Cu) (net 6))
 (segment (start 116.1 76.625) (end 116.1 77.7375) (width 0.25) (layer F.Cu) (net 6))
 (segment (start 112 78.54) (end 112.849999 77.690001) (width 0.25) (layer F.Cu) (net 6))
 (segment (start 112.849999 77.690001) (end 116.052501 77.690001) (width 0.25) (layer F.Cu) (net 6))
 (segment (start 116.052501 77.690001) (end 116.4875 78.125) (width 0.25) (layer F.Cu) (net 6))
 (segment (start 115.075 78.775) (end 114.9 78.6) (width 0.25) (layer F.Cu) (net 5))
 (segment (start 116.4875 78.775) (end 115.075 78.775) (width 0.25) (layer F.Cu) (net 5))
 (via (at 114.9 78.6) (size 0.8) (drill 0.4) (layers F.Cu B.Cu) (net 5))
 (segment (start 112.3 76) (end 112 76) (width 0.25) (layer B.Cu) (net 5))
 (segment (start 114.9 78.6) (end 112.3 76) (width 0.25) (layer B.Cu) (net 5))
 (segment (start 112.625 76.625) (end 112 76) (width 0.25) (layer F.Cu) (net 5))
 (segment (start 114.5 76.625) (end 112.625 76.625) (width 0.25) (layer F.Cu) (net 5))
 (segment (start 121.025 82.25) (end 120.875 82.1) (width 0.25) (layer F.Cu) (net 2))
 (segment (start 123 82.25) (end 121.025 82.25) (width 0.25) (layer F.Cu) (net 2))
 (segment (start 120.7125 81.9375) (end 120.875 82.1) (width 0.25) (layer F.Cu) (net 2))
 (segment (start 120.7125 80.075) (end 120.7125 81.9375) (width 0.25) (layer F.Cu) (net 2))
 (via (at 122.3 78.6) (size 0.8) (drill 0.4) (layers F.Cu B.Cu) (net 8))
 (segment (start 122.125 78.775) (end 122.3 78.6) (width 0.25) (layer F.Cu) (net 8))
 (segment (start 120.7125 78.775) (end 122.125 78.775) (width 0.25) (layer F.Cu) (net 8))
 (via (at 124.474697 79.077591) (size 0.8) (drill 0.4) (layers F.Cu B.Cu) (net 8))
 (segment (start 123.997106 78.6) (end 124.474697 79.077591) (width 0.25) (layer B.Cu) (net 8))
 (segment (start 122.3 78.6) (end 123.997106 78.6) (width 0.25) (layer B.Cu) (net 8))
 (segment (start 125.197591 79.077591) (end 126.12 80) (width 0.25) (layer F.Cu) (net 8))
 (segment (start 124.474697 79.077591) (end 125.197591 79.077591) (width 0.25) (layer F.Cu) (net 8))
 (segment (start 114.875 79.425) (end 114.3 80) (width 0.25) (layer F.Cu) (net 4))
 (segment (start 116.4875 79.425) (end 114.875 79.425) (width 0.25) (layer F.Cu) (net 4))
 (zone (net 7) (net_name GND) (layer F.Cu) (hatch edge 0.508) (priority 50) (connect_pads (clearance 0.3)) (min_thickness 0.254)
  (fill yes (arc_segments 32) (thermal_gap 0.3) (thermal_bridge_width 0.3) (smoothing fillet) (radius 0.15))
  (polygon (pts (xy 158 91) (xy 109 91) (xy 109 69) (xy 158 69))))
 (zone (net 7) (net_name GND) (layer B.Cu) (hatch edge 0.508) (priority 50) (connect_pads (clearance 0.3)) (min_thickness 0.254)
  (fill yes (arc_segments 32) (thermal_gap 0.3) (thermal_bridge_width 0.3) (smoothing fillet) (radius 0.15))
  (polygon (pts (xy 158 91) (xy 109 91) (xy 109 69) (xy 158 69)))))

